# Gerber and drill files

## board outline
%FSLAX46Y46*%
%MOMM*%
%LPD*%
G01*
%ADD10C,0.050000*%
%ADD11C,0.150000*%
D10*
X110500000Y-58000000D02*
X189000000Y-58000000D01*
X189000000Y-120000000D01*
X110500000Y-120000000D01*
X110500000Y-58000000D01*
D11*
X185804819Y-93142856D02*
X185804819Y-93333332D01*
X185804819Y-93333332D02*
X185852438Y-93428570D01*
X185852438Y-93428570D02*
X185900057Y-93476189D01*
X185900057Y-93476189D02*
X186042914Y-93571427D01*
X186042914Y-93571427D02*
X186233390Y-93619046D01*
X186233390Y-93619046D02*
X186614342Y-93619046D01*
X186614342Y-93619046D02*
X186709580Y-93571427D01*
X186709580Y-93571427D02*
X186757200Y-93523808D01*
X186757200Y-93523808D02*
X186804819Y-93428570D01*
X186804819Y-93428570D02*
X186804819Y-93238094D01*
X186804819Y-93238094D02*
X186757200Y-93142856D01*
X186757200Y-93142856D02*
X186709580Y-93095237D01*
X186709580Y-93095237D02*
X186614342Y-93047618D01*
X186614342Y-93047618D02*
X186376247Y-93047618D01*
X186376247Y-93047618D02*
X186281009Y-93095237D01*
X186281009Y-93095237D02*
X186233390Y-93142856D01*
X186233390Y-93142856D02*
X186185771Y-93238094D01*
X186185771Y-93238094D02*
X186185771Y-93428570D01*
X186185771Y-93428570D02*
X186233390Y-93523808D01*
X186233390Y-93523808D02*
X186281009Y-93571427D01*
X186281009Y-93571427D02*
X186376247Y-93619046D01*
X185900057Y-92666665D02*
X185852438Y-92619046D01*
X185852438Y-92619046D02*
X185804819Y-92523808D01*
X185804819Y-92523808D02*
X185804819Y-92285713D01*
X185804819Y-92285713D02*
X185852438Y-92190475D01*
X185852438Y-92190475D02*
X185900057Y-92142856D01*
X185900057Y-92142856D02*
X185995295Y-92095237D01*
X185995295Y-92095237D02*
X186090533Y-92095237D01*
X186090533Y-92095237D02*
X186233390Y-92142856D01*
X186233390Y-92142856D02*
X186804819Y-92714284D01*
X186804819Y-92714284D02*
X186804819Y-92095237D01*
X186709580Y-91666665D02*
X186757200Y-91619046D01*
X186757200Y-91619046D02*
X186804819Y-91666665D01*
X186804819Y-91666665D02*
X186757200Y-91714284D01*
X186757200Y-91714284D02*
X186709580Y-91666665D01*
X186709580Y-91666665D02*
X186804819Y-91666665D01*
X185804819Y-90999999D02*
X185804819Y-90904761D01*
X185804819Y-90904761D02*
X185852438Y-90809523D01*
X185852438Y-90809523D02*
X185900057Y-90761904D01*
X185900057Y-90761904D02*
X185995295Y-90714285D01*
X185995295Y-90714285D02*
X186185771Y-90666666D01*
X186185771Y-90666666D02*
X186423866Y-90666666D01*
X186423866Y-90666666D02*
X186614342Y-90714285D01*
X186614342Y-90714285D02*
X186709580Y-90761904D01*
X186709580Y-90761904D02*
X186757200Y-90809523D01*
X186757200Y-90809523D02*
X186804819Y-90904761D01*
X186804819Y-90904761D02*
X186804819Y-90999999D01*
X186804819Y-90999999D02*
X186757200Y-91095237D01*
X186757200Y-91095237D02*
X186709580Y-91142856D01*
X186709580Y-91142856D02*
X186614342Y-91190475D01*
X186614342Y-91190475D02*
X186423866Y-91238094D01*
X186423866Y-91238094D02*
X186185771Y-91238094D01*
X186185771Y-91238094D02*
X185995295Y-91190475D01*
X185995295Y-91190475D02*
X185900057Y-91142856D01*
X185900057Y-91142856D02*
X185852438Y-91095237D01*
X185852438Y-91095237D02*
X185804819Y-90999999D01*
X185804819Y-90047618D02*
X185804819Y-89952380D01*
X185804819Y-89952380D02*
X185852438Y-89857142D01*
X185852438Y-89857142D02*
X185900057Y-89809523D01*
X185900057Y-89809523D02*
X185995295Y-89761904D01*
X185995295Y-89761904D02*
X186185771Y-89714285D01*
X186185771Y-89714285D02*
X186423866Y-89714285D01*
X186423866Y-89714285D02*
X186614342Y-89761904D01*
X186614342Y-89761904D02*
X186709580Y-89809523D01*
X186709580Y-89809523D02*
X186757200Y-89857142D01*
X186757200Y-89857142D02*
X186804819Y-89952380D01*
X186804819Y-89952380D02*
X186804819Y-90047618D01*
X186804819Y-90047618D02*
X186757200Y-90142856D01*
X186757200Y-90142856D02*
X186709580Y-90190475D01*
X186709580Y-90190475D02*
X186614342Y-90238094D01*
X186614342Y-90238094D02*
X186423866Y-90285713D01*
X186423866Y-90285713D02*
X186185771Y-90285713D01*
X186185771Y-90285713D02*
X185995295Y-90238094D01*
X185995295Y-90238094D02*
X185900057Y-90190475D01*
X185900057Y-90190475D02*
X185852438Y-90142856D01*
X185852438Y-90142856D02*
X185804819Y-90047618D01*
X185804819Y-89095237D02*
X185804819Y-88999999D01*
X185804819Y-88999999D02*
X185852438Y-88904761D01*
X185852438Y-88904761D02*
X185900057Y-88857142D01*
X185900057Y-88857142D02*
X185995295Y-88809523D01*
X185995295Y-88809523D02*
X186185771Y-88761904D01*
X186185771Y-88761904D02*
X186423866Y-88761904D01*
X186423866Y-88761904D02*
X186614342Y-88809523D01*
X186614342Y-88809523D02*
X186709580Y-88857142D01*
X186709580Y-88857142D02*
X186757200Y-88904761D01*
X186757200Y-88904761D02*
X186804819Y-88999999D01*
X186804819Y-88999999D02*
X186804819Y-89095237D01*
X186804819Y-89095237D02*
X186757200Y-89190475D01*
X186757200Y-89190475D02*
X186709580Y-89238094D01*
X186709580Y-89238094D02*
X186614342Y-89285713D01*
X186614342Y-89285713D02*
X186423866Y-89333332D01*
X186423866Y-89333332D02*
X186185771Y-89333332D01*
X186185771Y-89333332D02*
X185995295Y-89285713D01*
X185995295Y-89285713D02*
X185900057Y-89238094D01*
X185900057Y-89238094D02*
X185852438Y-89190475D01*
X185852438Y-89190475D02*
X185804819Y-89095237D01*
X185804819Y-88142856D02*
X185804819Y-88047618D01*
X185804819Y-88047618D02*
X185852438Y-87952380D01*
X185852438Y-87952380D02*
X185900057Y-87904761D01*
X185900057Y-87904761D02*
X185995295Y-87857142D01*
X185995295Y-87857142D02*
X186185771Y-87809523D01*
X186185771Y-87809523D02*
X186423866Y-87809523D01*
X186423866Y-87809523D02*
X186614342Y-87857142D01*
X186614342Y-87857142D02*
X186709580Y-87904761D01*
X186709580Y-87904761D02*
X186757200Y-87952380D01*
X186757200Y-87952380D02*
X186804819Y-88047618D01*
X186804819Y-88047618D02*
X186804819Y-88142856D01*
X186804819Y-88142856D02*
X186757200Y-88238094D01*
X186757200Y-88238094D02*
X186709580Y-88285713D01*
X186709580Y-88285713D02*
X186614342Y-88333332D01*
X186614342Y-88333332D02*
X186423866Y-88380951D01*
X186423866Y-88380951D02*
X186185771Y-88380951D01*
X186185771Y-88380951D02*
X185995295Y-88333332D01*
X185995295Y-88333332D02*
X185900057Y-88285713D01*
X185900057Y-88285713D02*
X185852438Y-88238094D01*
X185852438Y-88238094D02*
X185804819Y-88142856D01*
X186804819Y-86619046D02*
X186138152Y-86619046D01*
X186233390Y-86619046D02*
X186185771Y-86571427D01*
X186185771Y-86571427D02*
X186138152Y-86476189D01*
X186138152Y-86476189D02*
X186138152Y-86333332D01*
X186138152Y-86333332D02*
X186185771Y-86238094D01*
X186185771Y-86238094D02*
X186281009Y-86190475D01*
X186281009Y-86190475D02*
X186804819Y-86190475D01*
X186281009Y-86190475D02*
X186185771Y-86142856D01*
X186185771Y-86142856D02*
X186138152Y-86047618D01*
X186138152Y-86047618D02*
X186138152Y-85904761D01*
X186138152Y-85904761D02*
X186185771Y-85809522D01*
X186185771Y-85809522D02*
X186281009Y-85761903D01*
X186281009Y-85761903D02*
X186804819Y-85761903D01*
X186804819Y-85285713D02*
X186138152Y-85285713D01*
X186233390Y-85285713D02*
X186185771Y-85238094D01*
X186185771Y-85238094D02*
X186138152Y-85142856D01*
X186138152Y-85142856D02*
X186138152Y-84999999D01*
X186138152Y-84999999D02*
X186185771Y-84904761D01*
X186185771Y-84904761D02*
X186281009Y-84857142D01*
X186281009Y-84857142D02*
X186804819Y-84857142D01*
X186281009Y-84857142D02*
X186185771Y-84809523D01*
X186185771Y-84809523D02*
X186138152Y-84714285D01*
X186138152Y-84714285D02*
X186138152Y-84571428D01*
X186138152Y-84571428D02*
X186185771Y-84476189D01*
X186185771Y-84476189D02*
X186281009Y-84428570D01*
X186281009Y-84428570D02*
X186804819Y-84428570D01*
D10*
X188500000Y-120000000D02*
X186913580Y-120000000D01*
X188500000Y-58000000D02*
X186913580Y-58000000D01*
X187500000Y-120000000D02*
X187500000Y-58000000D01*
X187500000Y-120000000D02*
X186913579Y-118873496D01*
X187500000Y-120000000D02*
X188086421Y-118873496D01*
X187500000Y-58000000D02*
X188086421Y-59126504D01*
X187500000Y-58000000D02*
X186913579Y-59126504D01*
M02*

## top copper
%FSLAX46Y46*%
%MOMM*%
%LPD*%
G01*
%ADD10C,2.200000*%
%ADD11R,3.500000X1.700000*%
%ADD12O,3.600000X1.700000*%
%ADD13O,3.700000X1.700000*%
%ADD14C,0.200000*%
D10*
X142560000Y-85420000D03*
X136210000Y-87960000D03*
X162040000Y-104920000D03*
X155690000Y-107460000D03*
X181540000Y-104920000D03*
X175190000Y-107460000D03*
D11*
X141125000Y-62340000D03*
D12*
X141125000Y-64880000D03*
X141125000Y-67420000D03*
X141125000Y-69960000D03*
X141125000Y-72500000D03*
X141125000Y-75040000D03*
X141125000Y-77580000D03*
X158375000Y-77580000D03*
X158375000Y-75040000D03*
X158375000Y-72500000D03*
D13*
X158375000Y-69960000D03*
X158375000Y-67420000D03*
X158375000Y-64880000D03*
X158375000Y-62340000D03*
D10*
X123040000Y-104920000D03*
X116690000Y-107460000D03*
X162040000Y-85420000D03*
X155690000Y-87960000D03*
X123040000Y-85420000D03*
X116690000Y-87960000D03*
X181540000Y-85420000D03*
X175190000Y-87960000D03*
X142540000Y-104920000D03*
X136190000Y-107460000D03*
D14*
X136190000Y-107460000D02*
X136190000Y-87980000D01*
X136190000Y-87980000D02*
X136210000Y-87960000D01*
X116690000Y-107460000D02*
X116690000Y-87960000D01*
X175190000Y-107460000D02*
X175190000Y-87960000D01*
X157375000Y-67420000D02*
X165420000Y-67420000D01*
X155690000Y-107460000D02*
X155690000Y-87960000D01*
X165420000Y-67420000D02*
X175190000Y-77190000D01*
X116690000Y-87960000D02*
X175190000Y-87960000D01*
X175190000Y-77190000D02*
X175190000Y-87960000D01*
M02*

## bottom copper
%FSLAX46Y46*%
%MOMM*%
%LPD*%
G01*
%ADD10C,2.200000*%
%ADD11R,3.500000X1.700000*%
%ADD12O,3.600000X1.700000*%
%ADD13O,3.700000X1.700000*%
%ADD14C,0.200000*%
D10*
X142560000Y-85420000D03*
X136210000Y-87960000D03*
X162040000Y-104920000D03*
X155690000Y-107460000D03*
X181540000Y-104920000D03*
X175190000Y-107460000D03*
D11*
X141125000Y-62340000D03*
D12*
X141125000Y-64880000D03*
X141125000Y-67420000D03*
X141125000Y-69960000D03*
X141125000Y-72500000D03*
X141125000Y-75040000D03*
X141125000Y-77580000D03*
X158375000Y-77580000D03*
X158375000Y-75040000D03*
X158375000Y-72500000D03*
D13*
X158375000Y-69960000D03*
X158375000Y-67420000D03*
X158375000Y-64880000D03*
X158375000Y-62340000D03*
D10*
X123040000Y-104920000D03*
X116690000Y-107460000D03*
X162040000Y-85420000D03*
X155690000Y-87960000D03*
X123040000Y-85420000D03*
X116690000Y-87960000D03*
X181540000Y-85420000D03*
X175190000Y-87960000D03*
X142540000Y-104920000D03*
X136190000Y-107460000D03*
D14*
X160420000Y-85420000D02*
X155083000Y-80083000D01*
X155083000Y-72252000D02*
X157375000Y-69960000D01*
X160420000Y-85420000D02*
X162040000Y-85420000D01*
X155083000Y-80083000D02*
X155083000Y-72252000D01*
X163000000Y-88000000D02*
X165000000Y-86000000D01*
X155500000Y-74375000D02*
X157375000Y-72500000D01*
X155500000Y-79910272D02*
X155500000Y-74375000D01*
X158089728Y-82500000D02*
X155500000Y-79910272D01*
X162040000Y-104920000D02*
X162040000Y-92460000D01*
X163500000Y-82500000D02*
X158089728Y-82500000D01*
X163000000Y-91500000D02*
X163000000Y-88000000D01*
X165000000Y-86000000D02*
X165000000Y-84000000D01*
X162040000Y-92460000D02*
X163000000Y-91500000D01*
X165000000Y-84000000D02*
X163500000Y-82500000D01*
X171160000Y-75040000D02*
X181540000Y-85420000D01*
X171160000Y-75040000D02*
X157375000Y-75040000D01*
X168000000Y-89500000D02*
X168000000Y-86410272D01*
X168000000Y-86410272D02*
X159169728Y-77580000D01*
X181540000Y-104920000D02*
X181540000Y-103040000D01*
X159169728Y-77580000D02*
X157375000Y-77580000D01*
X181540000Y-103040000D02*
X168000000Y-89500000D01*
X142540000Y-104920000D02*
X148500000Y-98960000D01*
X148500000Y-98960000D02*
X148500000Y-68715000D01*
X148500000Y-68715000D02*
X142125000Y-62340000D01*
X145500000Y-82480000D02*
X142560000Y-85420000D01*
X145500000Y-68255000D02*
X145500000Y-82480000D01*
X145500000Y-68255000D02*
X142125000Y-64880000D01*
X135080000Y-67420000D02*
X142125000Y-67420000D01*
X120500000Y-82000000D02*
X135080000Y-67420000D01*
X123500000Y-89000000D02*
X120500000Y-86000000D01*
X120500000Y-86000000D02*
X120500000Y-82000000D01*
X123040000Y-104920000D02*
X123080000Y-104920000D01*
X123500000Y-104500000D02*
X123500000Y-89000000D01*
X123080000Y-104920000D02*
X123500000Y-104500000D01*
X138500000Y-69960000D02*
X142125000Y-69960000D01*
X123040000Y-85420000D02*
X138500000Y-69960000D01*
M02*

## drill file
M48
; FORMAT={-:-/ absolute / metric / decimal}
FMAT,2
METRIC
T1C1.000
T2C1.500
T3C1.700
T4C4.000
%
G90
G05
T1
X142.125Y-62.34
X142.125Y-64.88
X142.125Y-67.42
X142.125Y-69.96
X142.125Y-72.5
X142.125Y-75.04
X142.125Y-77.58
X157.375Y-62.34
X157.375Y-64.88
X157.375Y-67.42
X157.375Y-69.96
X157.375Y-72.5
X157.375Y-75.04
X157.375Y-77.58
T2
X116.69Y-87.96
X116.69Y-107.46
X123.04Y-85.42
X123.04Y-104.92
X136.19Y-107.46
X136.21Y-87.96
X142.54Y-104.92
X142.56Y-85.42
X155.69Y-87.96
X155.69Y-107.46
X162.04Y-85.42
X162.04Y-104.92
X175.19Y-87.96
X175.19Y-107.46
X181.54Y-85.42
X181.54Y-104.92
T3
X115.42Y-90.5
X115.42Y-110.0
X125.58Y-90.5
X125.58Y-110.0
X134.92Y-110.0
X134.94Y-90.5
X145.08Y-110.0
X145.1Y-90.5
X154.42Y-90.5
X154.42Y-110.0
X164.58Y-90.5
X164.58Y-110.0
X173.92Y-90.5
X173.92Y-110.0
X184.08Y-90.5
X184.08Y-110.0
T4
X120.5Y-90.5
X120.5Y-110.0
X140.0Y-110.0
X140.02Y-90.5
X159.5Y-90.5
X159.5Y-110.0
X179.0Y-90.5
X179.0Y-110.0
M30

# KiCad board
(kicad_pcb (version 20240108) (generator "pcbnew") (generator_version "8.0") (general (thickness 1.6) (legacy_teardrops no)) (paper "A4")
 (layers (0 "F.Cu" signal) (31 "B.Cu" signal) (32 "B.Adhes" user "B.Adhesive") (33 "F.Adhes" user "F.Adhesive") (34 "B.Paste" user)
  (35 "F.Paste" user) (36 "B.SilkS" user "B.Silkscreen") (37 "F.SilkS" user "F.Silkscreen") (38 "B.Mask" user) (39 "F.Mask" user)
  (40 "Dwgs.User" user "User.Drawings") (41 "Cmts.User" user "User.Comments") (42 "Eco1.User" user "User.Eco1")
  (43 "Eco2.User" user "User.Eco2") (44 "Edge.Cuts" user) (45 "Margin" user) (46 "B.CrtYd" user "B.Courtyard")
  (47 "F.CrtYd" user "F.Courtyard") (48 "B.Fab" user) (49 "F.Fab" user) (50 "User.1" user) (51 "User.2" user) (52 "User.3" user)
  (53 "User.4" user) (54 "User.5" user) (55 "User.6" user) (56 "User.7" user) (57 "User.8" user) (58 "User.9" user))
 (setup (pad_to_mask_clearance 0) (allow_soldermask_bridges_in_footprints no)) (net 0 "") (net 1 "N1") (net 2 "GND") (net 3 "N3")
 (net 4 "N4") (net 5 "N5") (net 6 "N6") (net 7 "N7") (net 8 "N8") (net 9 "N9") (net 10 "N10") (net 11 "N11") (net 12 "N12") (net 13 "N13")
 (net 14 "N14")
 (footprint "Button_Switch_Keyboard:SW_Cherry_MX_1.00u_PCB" (layer "F.Cu") (at 142.54 85.42)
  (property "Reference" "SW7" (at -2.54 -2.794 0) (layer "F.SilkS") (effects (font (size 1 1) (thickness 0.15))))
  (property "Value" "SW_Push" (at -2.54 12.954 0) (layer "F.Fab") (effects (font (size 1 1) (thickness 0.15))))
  (pad "" np_thru_hole circle (at -7.6 5.08) (size 1.7 1.7) (drill 1.7) (layers "*.Cu" "*.Mask"))
  (pad "" np_thru_hole circle (at -2.52 5.08) (size 4 4) (drill 4) (layers "*.Cu" "*.Mask"))
  (pad "" np_thru_hole circle (at 2.56 5.08) (size 1.7 1.7) (drill 1.7) (layers "*.Cu" "*.Mask"))
  (pad "1" thru_hole circle (at 0.02 0) (size 2.2 2.2) (drill 1.5) (layers "*.Cu" "*.Mask") (remove_unused_layers no) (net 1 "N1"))
  (pad "2" thru_hole circle (at -6.33 2.54) (size 2.2 2.2) (drill 1.5) (layers "*.Cu" "*.Mask") (remove_unused_layers no) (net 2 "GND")))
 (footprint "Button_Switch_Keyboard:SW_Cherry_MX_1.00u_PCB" (layer "F.Cu") (at 162.04 104.92)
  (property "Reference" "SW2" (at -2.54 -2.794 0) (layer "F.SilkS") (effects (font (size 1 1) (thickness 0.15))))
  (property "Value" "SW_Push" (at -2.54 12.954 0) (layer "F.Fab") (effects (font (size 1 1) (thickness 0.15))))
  (pad "" np_thru_hole circle (at -7.62 5.08) (size 1.7 1.7) (drill 1.7) (layers "*.Cu" "*.Mask"))
  (pad "" np_thru_hole circle (at -2.54 5.08) (size 4 4) (drill 4) (layers "*.Cu" "*.Mask"))
  (pad "" np_thru_hole circle (at 2.54 5.08) (size 1.7 1.7) (drill 1.7) (layers "*.Cu" "*.Mask"))
  (pad "1" thru_hole circle (at 0 0) (size 2.2 2.2) (drill 1.5) (layers "*.Cu" "*.Mask") (remove_unused_layers no) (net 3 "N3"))
  (pad "2" thru_hole circle (at -6.35 2.54) (size 2.2 2.2) (drill 1.5) (layers "*.Cu" "*.Mask") (remove_unused_layers no) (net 2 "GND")))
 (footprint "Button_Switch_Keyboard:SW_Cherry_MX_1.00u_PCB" (layer "F.Cu") (at 181.54 104.92)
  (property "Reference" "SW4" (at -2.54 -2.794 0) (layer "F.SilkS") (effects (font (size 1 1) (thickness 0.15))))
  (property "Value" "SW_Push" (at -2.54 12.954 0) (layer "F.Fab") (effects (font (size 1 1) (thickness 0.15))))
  (pad "" np_thru_hole circle (at -7.62 5.08) (size 1.7 1.7) (drill 1.7) (layers "*.Cu" "*.Mask"))
  (pad "" np_thru_hole circle (at -2.54 5.08) (size 4 4) (drill 4) (layers "*.Cu" "*.Mask"))
  (pad "" np_thru_hole circle (at 2.54 5.08) (size 1.7 1.7) (drill 1.7) (layers "*.Cu" "*.Mask"))
  (pad "1" thru_hole circle (at 0 0) (size 2.2 2.2) (drill 1.5) (layers "*.Cu" "*.Mask") (remove_unused_layers no) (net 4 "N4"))
  (pad "2" thru_hole circle (at -6.35 2.54) (size 2.2 2.2) (drill 1.5) (layers "*.Cu" "*.Mask") (remove_unused_layers no) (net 2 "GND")))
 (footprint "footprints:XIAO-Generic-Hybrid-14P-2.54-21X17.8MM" (layer "F.Cu") (at 149.75 69.96)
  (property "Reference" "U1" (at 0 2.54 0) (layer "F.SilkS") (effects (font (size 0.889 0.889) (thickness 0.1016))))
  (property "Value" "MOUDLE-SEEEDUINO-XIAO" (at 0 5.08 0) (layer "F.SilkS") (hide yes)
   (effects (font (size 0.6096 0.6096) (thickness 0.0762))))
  (pad "1" thru_hole rect (at -7.625 -7.62) (size 3.5 1.7) (drill 1 (offset -1 0)) (layers "*.Cu" "*.Mask") (remove_unused_layers no)
   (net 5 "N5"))
  (pad "2" thru_hole oval (at -7.625 -5.08) (size 3.6 1.7) (drill 1 (offset -1 0)) (layers "*.Cu" "*.Mask") (remove_unused_layers no)
   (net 1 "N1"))
  (pad "3" thru_hole oval (at -7.625 -2.54) (size 3.6 1.7) (drill 1 (offset -1 0)) (layers "*.Cu" "*.Mask") (remove_unused_layers no)
   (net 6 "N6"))
  (pad "4" thru_hole oval (at -7.625 0) (size 3.6 1.7) (drill 1 (offset -1 0)) (layers "*.Cu" "*.Mask") (remove_unused_layers no)
   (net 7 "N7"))
  (pad "5" thru_hole oval (at -7.625 2.54) (size 3.6 1.7) (drill 1 (offset -1 0)) (layers "*.Cu" "*.Mask") (remove_unused_layers no)
   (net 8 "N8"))
  (pad "6" thru_hole oval (at -7.625 5.08 180) (size 3.6 1.7) (drill 1 (offset 1 0)) (layers "*.Cu" "*.Mask") (remove_unused_layers no)
   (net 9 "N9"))
  (pad "7" thru_hole oval (at -7.625 7.62) (size 3.6 1.7) (drill 1 (offset -1 0)) (layers "*.Cu" "*.Mask") (remove_unused_layers no)
   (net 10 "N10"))
  (pad "8" thru_hole oval (at 7.625 7.62) (size 3.6 1.7) (drill 1 (offset 1 0)) (layers "*.Cu" "*.Mask") (remove_unused_layers no)
   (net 4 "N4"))
  (pad "9" thru_hole oval (at 7.625 5.08) (size 3.6 1.7) (drill 1 (offset 1 0)) (layers "*.Cu" "*.Mask") (remove_unused_layers no)
   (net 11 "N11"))
  (pad "10" thru_hole oval (at 7.625 2.54) (size 3.6 1.7) (drill 1 (offset 1 0)) (layers "*.Cu" "*.Mask") (remove_unused_layers no)
   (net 3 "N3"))
  (pad "11" thru_hole oval (at 7.625 0) (size 3.7 1.7) (drill 1 (offset 1 0)) (layers "*.Cu" "*.Mask") (remove_unused_layers no)
   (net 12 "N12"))
  (pad "12" thru_hole oval (at 7.625 -2.54) (size 3.7 1.7) (drill 1 (offset 1 0)) (layers "*.Cu" "*.Mask") (remove_unused_layers no)
   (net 2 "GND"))
  (pad "13" thru_hole oval (at 7.625 -5.08) (size 3.7 1.7) (drill 1 (offset 1 0)) (layers "*.Cu" "*.Mask") (remove_unused_layers no)
   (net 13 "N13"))
  (pad "14" thru_hole oval (at 7.625 -7.62) (size 3.7 1.7) (drill 1 (offset 1 0)) (layers "*.Cu" "*.Mask") (remove_unused_layers no)
   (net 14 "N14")))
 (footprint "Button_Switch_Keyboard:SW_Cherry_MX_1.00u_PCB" (layer "F.Cu") (at 123.04 104.92)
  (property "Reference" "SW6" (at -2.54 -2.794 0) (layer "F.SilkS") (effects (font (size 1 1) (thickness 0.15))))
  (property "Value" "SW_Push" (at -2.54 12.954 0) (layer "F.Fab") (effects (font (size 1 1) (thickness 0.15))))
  (pad "" np_thru_hole circle (at -7.62 5.08) (size 1.7 1.7) (drill 1.7) (layers "*.Cu" "*.Mask"))
  (pad "" np_thru_hole circle (at -2.54 5.08) (size 4 4) (drill 4) (layers "*.Cu" "*.Mask"))
  (pad "" np_thru_hole circle (at 2.54 5.08) (size 1.7 1.7) (drill 1.7) (layers "*.Cu" "*.Mask"))
  (pad "1" thru_hole circle (at 0 0) (size 2.2 2.2) (drill 1.5) (layers "*.Cu" "*.Mask") (remove_unused_layers no) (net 6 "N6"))
  (pad "2" thru_hole circle (at -6.35 2.54) (size 2.2 2.2) (drill 1.5) (layers "*.Cu" "*.Mask") (remove_unused_layers no) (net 2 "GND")))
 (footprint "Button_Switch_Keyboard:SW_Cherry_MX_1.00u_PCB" (layer "F.Cu") (at 162.04 85.42)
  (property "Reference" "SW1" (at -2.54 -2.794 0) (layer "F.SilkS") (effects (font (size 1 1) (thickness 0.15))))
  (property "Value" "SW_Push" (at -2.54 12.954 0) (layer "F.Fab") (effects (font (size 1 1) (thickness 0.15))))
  (pad "" np_thru_hole circle (at -7.62 5.08) (size 1.7 1.7) (drill 1.7) (layers "*.Cu" "*.Mask"))
  (pad "" np_thru_hole circle (at -2.54 5.08) (size 4 4) (drill 4) (layers "*.Cu" "*.Mask"))
  (pad "" np_thru_hole circle (at 2.54 5.08) (size 1.7 1.7) (drill 1.7) (layers "*.Cu" "*.Mask"))
  (pad "1" thru_hole circle (at 0 0) (size 2.2 2.2) (drill 1.5) (layers "*.Cu" "*.Mask") (remove_unused_layers no) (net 12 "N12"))
  (pad "2" thru_hole circle (at -6.35 2.54) (size 2.2 2.2) (drill 1.5) (layers "*.Cu" "*.Mask") (remove_unused_layers no) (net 2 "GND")))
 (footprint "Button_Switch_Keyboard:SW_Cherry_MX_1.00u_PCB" (layer "F.Cu") (at 123.04 85.42)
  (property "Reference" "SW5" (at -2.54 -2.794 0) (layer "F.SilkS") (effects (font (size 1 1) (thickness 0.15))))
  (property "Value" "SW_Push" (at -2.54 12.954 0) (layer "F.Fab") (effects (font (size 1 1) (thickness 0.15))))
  (pad "" np_thru_hole circle (at -7.62 5.08) (size 1.7 1.7) (drill 1.7) (layers "*.Cu" "*.Mask"))
  (pad "" np_thru_hole circle (at -2.54 5.08) (size 4 4) (drill 4) (layers "*.Cu" "*.Mask"))
  (pad "" np_thru_hole circle (at 2.54 5.08) (size 1.7 1.7) (drill 1.7) (layers "*.Cu" "*.Mask"))
  (pad "1" thru_hole circle (at 0 0) (size 2.2 2.2) (drill 1.5) (layers "*.Cu" "*.Mask") (remove_unused_layers no) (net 7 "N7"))
  (pad "2" thru_hole circle (at -6.35 2.54) (size 2.2 2.2) (drill 1.5) (layers "*.Cu" "*.Mask") (remove_unused_layers no) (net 2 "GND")))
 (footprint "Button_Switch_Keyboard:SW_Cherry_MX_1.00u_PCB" (layer "F.Cu") (at 181.54 85.42)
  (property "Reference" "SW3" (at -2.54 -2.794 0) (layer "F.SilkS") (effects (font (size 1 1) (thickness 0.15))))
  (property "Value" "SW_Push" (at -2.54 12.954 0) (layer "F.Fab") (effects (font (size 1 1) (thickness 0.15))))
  (pad "" np_thru_hole circle (at -7.62 5.08) (size 1.7 1.7) (drill 1.7) (layers "*.Cu" "*.Mask"))
  (pad "" np_thru_hole circle (at -2.54 5.08) (size 4 4) (drill 4) (layers "*.Cu" "*.Mask"))
  (pad "" np_thru_hole circle (at 2.54 5.08) (size 1.7 1.7) (drill 1.7) (layers "*.Cu" "*.Mask"))
  (pad "1" thru_hole circle (at 0 0) (size 2.2 2.2) (drill 1.5) (layers "*.Cu" "*.Mask") (remove_unused_layers no) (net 11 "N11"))
  (pad "2" thru_hole circle (at -6.35 2.54) (size 2.2 2.2) (drill 1.5) (layers "*.Cu" "*.Mask") (remove_unused_layers no) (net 2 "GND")))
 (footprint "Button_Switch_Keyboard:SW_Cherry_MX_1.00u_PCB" (layer "F.Cu") (at 142.54 104.92)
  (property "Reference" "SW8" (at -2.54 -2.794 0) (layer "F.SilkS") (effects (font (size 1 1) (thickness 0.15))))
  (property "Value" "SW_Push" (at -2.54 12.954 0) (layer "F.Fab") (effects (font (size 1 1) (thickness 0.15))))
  (pad "" np_thru_hole circle (at -7.62 5.08) (size 1.7 1.7) (drill 1.7) (layers "*.Cu" "*.Mask"))
  (pad "" np_thru_hole circle (at -2.54 5.08) (size 4 4) (drill 4) (layers "*.Cu" "*.Mask"))
  (pad "" np_thru_hole circle (at 2.54 5.08) (size 1.7 1.7) (drill 1.7) (layers "*.Cu" "*.Mask"))
  (pad "1" thru_hole circle (at 0 0) (size 2.2 2.2) (drill 1.5) (layers "*.Cu" "*.Mask") (remove_unused_layers no) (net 5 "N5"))
  (pad "2" thru_hole circle (at -6.35 2.54) (size 2.2 2.2) (drill 1.5) (layers "*.Cu" "*.Mask") (remove_unused_layers no) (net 2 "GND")))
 (gr_rect (start 110.5 58) (end 189 120) (stroke (width 0.05) (type default)) (fill none) (layer "Edge.Cuts"))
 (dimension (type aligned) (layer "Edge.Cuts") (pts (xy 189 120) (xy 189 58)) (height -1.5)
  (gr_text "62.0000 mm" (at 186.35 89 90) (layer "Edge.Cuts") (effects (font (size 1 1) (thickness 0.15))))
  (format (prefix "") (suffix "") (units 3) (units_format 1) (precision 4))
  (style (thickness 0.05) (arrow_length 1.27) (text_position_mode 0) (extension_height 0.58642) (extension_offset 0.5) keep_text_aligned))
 (segment (start 136.19 107.46) (end 136.19 87.98) (width 0.2) (layer "F.Cu") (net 2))
 (segment (start 136.19 87.98) (end 136.21 87.96) (width 0.2) (layer "F.Cu") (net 2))
 (segment (start 116.69 107.46) (end 116.69 87.96) (width 0.2) (layer "F.Cu") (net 2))
 (segment (start 175.19 107.46) (end 175.19 87.96) (width 0.2) (layer "F.Cu") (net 2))
 (segment (start 157.375 67.42) (end 165.42 67.42) (width 0.2) (layer "F.Cu") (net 2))
 (segment (start 155.69 107.46) (end 155.69 87.96) (width 0.2) (layer "F.Cu") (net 2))
 (segment (start 165.42 67.42) (end 175.19 77.19) (width 0.2) (layer "F.Cu") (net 2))
 (segment (start 116.69 87.96) (end 175.19 87.96) (width 0.2) (layer "F.Cu") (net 2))
 (segment (start 175.19 77.19) (end 175.19 87.96) (width 0.2) (layer "F.Cu") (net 2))
 (segment (start 160.42 85.42) (end 155.083 80.083) (width 0.2) (layer "B.Cu") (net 12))
 (segment (start 155.083 72.252) (end 157.375 69.96) (width 0.2) (layer "B.Cu") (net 12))
 (segment (start 160.42 85.42) (end 162.04 85.42) (width 0.2) (layer "B.Cu") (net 12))
 (segment (start 155.083 80.083) (end 155.083 72.252) (width 0.2) (layer "B.Cu") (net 12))
 (segment (start 163 88) (end 165 86) (width 0.2) (layer "B.Cu") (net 3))
 (segment (start 155.5 74.375) (end 157.375 72.5) (width 0.2) (layer "B.Cu") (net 3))
 (segment (start 155.5 79.910272) (end 155.5 74.375) (width 0.2) (layer "B.Cu") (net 3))
 (segment (start 158.089728 82.5) (end 155.5 79.910272) (width 0.2) (layer "B.Cu") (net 3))
 (segment (start 162.04 104.92) (end 162.04 92.46) (width 0.2) (layer "B.Cu") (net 3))
 (segment (start 163.5 82.5) (end 158.089728 82.5) (width 0.2) (layer "B.Cu") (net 3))
 (segment (start 163 91.5) (end 163 88) (width 0.2) (layer "B.Cu") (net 3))
 (segment (start 165 86) (end 165 84) (width 0.2) (layer "B.Cu") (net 3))
 (segment (start 162.04 92.46) (end 163 91.5) (width 0.2) (layer "B.Cu") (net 3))
 (segment (start 165 84) (end 163.5 82.5) (width 0.2) (layer "B.Cu") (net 3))
 (segment (start 171.16 75.04) (end 181.54 85.42) (width 0.2) (layer "B.Cu") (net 11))
 (segment (start 171.16 75.04) (end 157.375 75.04) (width 0.2) (layer "B.Cu") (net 11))
 (segment (start 168 89.5) (end 168 86.410272) (width 0.2) (layer "B.Cu") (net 4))
 (segment (start 168 86.410272) (end 159.169728 77.58) (width 0.2) (layer "B.Cu") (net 4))
 (segment (start 181.54 104.92) (end 181.54 103.04) (width 0.2) (layer "B.Cu") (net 4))
 (segment (start 159.169728 77.58) (end 157.375 77.58) (width 0.2) (layer "B.Cu") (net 4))
 (segment (start 181.54 103.04) (end 168 89.5) (width 0.2) (layer "B.Cu") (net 4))
 (segment (start 142.54 104.92) (end 148.5 98.96) (width 0.2) (layer "B.Cu") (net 5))
 (segment (start 148.5 98.96) (end 148.5 68.715) (width 0.2) (layer "B.Cu") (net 5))
 (segment (start 148.5 68.715) (end 142.125 62.34) (width 0.2) (layer "B.Cu") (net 5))
 (segment (start 145.5 82.48) (end 142.56 85.42) (width 0.2) (layer "B.Cu") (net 1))
 (segment (start 145.5 68.255) (end 145.5 82.48) (width 0.2) (layer "B.Cu") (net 1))
 (segment (start 145.5 68.255) (end 142.125 64.88) (width 0.2) (layer "B.Cu") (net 1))
 (segment (start 135.08 67.42) (end 142.125 67.42) (width 0.2) (layer "B.Cu") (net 6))
 (segment (start 120.5 82) (end 135.08 67.42) (width 0.2) (layer "B.Cu") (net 6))
 (segment (start 123.5 89) (end 120.5 86) (width 0.2) (layer "B.Cu") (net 6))
 (segment (start 120.5 86) (end 120.5 82) (width 0.2) (layer "B.Cu") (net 6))
 (segment (start 123.04 104.92) (end 123.08 104.92) (width 0.2) (layer "B.Cu") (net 6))
 (segment (start 123.5 104.5) (end 123.5 89) (width 0.2) (layer "B.Cu") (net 6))
 (segment (start 123.08 104.92) (end 123.5 104.5) (width 0.2) (layer "B.Cu") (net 6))
 (segment (start 138.5 69.96) (end 142.125 69.96) (width 0.2) (layer "B.Cu") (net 7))
 (segment (start 123.04 85.42) (end 138.5 69.96) (width 0.2) (layer "B.Cu") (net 7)))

